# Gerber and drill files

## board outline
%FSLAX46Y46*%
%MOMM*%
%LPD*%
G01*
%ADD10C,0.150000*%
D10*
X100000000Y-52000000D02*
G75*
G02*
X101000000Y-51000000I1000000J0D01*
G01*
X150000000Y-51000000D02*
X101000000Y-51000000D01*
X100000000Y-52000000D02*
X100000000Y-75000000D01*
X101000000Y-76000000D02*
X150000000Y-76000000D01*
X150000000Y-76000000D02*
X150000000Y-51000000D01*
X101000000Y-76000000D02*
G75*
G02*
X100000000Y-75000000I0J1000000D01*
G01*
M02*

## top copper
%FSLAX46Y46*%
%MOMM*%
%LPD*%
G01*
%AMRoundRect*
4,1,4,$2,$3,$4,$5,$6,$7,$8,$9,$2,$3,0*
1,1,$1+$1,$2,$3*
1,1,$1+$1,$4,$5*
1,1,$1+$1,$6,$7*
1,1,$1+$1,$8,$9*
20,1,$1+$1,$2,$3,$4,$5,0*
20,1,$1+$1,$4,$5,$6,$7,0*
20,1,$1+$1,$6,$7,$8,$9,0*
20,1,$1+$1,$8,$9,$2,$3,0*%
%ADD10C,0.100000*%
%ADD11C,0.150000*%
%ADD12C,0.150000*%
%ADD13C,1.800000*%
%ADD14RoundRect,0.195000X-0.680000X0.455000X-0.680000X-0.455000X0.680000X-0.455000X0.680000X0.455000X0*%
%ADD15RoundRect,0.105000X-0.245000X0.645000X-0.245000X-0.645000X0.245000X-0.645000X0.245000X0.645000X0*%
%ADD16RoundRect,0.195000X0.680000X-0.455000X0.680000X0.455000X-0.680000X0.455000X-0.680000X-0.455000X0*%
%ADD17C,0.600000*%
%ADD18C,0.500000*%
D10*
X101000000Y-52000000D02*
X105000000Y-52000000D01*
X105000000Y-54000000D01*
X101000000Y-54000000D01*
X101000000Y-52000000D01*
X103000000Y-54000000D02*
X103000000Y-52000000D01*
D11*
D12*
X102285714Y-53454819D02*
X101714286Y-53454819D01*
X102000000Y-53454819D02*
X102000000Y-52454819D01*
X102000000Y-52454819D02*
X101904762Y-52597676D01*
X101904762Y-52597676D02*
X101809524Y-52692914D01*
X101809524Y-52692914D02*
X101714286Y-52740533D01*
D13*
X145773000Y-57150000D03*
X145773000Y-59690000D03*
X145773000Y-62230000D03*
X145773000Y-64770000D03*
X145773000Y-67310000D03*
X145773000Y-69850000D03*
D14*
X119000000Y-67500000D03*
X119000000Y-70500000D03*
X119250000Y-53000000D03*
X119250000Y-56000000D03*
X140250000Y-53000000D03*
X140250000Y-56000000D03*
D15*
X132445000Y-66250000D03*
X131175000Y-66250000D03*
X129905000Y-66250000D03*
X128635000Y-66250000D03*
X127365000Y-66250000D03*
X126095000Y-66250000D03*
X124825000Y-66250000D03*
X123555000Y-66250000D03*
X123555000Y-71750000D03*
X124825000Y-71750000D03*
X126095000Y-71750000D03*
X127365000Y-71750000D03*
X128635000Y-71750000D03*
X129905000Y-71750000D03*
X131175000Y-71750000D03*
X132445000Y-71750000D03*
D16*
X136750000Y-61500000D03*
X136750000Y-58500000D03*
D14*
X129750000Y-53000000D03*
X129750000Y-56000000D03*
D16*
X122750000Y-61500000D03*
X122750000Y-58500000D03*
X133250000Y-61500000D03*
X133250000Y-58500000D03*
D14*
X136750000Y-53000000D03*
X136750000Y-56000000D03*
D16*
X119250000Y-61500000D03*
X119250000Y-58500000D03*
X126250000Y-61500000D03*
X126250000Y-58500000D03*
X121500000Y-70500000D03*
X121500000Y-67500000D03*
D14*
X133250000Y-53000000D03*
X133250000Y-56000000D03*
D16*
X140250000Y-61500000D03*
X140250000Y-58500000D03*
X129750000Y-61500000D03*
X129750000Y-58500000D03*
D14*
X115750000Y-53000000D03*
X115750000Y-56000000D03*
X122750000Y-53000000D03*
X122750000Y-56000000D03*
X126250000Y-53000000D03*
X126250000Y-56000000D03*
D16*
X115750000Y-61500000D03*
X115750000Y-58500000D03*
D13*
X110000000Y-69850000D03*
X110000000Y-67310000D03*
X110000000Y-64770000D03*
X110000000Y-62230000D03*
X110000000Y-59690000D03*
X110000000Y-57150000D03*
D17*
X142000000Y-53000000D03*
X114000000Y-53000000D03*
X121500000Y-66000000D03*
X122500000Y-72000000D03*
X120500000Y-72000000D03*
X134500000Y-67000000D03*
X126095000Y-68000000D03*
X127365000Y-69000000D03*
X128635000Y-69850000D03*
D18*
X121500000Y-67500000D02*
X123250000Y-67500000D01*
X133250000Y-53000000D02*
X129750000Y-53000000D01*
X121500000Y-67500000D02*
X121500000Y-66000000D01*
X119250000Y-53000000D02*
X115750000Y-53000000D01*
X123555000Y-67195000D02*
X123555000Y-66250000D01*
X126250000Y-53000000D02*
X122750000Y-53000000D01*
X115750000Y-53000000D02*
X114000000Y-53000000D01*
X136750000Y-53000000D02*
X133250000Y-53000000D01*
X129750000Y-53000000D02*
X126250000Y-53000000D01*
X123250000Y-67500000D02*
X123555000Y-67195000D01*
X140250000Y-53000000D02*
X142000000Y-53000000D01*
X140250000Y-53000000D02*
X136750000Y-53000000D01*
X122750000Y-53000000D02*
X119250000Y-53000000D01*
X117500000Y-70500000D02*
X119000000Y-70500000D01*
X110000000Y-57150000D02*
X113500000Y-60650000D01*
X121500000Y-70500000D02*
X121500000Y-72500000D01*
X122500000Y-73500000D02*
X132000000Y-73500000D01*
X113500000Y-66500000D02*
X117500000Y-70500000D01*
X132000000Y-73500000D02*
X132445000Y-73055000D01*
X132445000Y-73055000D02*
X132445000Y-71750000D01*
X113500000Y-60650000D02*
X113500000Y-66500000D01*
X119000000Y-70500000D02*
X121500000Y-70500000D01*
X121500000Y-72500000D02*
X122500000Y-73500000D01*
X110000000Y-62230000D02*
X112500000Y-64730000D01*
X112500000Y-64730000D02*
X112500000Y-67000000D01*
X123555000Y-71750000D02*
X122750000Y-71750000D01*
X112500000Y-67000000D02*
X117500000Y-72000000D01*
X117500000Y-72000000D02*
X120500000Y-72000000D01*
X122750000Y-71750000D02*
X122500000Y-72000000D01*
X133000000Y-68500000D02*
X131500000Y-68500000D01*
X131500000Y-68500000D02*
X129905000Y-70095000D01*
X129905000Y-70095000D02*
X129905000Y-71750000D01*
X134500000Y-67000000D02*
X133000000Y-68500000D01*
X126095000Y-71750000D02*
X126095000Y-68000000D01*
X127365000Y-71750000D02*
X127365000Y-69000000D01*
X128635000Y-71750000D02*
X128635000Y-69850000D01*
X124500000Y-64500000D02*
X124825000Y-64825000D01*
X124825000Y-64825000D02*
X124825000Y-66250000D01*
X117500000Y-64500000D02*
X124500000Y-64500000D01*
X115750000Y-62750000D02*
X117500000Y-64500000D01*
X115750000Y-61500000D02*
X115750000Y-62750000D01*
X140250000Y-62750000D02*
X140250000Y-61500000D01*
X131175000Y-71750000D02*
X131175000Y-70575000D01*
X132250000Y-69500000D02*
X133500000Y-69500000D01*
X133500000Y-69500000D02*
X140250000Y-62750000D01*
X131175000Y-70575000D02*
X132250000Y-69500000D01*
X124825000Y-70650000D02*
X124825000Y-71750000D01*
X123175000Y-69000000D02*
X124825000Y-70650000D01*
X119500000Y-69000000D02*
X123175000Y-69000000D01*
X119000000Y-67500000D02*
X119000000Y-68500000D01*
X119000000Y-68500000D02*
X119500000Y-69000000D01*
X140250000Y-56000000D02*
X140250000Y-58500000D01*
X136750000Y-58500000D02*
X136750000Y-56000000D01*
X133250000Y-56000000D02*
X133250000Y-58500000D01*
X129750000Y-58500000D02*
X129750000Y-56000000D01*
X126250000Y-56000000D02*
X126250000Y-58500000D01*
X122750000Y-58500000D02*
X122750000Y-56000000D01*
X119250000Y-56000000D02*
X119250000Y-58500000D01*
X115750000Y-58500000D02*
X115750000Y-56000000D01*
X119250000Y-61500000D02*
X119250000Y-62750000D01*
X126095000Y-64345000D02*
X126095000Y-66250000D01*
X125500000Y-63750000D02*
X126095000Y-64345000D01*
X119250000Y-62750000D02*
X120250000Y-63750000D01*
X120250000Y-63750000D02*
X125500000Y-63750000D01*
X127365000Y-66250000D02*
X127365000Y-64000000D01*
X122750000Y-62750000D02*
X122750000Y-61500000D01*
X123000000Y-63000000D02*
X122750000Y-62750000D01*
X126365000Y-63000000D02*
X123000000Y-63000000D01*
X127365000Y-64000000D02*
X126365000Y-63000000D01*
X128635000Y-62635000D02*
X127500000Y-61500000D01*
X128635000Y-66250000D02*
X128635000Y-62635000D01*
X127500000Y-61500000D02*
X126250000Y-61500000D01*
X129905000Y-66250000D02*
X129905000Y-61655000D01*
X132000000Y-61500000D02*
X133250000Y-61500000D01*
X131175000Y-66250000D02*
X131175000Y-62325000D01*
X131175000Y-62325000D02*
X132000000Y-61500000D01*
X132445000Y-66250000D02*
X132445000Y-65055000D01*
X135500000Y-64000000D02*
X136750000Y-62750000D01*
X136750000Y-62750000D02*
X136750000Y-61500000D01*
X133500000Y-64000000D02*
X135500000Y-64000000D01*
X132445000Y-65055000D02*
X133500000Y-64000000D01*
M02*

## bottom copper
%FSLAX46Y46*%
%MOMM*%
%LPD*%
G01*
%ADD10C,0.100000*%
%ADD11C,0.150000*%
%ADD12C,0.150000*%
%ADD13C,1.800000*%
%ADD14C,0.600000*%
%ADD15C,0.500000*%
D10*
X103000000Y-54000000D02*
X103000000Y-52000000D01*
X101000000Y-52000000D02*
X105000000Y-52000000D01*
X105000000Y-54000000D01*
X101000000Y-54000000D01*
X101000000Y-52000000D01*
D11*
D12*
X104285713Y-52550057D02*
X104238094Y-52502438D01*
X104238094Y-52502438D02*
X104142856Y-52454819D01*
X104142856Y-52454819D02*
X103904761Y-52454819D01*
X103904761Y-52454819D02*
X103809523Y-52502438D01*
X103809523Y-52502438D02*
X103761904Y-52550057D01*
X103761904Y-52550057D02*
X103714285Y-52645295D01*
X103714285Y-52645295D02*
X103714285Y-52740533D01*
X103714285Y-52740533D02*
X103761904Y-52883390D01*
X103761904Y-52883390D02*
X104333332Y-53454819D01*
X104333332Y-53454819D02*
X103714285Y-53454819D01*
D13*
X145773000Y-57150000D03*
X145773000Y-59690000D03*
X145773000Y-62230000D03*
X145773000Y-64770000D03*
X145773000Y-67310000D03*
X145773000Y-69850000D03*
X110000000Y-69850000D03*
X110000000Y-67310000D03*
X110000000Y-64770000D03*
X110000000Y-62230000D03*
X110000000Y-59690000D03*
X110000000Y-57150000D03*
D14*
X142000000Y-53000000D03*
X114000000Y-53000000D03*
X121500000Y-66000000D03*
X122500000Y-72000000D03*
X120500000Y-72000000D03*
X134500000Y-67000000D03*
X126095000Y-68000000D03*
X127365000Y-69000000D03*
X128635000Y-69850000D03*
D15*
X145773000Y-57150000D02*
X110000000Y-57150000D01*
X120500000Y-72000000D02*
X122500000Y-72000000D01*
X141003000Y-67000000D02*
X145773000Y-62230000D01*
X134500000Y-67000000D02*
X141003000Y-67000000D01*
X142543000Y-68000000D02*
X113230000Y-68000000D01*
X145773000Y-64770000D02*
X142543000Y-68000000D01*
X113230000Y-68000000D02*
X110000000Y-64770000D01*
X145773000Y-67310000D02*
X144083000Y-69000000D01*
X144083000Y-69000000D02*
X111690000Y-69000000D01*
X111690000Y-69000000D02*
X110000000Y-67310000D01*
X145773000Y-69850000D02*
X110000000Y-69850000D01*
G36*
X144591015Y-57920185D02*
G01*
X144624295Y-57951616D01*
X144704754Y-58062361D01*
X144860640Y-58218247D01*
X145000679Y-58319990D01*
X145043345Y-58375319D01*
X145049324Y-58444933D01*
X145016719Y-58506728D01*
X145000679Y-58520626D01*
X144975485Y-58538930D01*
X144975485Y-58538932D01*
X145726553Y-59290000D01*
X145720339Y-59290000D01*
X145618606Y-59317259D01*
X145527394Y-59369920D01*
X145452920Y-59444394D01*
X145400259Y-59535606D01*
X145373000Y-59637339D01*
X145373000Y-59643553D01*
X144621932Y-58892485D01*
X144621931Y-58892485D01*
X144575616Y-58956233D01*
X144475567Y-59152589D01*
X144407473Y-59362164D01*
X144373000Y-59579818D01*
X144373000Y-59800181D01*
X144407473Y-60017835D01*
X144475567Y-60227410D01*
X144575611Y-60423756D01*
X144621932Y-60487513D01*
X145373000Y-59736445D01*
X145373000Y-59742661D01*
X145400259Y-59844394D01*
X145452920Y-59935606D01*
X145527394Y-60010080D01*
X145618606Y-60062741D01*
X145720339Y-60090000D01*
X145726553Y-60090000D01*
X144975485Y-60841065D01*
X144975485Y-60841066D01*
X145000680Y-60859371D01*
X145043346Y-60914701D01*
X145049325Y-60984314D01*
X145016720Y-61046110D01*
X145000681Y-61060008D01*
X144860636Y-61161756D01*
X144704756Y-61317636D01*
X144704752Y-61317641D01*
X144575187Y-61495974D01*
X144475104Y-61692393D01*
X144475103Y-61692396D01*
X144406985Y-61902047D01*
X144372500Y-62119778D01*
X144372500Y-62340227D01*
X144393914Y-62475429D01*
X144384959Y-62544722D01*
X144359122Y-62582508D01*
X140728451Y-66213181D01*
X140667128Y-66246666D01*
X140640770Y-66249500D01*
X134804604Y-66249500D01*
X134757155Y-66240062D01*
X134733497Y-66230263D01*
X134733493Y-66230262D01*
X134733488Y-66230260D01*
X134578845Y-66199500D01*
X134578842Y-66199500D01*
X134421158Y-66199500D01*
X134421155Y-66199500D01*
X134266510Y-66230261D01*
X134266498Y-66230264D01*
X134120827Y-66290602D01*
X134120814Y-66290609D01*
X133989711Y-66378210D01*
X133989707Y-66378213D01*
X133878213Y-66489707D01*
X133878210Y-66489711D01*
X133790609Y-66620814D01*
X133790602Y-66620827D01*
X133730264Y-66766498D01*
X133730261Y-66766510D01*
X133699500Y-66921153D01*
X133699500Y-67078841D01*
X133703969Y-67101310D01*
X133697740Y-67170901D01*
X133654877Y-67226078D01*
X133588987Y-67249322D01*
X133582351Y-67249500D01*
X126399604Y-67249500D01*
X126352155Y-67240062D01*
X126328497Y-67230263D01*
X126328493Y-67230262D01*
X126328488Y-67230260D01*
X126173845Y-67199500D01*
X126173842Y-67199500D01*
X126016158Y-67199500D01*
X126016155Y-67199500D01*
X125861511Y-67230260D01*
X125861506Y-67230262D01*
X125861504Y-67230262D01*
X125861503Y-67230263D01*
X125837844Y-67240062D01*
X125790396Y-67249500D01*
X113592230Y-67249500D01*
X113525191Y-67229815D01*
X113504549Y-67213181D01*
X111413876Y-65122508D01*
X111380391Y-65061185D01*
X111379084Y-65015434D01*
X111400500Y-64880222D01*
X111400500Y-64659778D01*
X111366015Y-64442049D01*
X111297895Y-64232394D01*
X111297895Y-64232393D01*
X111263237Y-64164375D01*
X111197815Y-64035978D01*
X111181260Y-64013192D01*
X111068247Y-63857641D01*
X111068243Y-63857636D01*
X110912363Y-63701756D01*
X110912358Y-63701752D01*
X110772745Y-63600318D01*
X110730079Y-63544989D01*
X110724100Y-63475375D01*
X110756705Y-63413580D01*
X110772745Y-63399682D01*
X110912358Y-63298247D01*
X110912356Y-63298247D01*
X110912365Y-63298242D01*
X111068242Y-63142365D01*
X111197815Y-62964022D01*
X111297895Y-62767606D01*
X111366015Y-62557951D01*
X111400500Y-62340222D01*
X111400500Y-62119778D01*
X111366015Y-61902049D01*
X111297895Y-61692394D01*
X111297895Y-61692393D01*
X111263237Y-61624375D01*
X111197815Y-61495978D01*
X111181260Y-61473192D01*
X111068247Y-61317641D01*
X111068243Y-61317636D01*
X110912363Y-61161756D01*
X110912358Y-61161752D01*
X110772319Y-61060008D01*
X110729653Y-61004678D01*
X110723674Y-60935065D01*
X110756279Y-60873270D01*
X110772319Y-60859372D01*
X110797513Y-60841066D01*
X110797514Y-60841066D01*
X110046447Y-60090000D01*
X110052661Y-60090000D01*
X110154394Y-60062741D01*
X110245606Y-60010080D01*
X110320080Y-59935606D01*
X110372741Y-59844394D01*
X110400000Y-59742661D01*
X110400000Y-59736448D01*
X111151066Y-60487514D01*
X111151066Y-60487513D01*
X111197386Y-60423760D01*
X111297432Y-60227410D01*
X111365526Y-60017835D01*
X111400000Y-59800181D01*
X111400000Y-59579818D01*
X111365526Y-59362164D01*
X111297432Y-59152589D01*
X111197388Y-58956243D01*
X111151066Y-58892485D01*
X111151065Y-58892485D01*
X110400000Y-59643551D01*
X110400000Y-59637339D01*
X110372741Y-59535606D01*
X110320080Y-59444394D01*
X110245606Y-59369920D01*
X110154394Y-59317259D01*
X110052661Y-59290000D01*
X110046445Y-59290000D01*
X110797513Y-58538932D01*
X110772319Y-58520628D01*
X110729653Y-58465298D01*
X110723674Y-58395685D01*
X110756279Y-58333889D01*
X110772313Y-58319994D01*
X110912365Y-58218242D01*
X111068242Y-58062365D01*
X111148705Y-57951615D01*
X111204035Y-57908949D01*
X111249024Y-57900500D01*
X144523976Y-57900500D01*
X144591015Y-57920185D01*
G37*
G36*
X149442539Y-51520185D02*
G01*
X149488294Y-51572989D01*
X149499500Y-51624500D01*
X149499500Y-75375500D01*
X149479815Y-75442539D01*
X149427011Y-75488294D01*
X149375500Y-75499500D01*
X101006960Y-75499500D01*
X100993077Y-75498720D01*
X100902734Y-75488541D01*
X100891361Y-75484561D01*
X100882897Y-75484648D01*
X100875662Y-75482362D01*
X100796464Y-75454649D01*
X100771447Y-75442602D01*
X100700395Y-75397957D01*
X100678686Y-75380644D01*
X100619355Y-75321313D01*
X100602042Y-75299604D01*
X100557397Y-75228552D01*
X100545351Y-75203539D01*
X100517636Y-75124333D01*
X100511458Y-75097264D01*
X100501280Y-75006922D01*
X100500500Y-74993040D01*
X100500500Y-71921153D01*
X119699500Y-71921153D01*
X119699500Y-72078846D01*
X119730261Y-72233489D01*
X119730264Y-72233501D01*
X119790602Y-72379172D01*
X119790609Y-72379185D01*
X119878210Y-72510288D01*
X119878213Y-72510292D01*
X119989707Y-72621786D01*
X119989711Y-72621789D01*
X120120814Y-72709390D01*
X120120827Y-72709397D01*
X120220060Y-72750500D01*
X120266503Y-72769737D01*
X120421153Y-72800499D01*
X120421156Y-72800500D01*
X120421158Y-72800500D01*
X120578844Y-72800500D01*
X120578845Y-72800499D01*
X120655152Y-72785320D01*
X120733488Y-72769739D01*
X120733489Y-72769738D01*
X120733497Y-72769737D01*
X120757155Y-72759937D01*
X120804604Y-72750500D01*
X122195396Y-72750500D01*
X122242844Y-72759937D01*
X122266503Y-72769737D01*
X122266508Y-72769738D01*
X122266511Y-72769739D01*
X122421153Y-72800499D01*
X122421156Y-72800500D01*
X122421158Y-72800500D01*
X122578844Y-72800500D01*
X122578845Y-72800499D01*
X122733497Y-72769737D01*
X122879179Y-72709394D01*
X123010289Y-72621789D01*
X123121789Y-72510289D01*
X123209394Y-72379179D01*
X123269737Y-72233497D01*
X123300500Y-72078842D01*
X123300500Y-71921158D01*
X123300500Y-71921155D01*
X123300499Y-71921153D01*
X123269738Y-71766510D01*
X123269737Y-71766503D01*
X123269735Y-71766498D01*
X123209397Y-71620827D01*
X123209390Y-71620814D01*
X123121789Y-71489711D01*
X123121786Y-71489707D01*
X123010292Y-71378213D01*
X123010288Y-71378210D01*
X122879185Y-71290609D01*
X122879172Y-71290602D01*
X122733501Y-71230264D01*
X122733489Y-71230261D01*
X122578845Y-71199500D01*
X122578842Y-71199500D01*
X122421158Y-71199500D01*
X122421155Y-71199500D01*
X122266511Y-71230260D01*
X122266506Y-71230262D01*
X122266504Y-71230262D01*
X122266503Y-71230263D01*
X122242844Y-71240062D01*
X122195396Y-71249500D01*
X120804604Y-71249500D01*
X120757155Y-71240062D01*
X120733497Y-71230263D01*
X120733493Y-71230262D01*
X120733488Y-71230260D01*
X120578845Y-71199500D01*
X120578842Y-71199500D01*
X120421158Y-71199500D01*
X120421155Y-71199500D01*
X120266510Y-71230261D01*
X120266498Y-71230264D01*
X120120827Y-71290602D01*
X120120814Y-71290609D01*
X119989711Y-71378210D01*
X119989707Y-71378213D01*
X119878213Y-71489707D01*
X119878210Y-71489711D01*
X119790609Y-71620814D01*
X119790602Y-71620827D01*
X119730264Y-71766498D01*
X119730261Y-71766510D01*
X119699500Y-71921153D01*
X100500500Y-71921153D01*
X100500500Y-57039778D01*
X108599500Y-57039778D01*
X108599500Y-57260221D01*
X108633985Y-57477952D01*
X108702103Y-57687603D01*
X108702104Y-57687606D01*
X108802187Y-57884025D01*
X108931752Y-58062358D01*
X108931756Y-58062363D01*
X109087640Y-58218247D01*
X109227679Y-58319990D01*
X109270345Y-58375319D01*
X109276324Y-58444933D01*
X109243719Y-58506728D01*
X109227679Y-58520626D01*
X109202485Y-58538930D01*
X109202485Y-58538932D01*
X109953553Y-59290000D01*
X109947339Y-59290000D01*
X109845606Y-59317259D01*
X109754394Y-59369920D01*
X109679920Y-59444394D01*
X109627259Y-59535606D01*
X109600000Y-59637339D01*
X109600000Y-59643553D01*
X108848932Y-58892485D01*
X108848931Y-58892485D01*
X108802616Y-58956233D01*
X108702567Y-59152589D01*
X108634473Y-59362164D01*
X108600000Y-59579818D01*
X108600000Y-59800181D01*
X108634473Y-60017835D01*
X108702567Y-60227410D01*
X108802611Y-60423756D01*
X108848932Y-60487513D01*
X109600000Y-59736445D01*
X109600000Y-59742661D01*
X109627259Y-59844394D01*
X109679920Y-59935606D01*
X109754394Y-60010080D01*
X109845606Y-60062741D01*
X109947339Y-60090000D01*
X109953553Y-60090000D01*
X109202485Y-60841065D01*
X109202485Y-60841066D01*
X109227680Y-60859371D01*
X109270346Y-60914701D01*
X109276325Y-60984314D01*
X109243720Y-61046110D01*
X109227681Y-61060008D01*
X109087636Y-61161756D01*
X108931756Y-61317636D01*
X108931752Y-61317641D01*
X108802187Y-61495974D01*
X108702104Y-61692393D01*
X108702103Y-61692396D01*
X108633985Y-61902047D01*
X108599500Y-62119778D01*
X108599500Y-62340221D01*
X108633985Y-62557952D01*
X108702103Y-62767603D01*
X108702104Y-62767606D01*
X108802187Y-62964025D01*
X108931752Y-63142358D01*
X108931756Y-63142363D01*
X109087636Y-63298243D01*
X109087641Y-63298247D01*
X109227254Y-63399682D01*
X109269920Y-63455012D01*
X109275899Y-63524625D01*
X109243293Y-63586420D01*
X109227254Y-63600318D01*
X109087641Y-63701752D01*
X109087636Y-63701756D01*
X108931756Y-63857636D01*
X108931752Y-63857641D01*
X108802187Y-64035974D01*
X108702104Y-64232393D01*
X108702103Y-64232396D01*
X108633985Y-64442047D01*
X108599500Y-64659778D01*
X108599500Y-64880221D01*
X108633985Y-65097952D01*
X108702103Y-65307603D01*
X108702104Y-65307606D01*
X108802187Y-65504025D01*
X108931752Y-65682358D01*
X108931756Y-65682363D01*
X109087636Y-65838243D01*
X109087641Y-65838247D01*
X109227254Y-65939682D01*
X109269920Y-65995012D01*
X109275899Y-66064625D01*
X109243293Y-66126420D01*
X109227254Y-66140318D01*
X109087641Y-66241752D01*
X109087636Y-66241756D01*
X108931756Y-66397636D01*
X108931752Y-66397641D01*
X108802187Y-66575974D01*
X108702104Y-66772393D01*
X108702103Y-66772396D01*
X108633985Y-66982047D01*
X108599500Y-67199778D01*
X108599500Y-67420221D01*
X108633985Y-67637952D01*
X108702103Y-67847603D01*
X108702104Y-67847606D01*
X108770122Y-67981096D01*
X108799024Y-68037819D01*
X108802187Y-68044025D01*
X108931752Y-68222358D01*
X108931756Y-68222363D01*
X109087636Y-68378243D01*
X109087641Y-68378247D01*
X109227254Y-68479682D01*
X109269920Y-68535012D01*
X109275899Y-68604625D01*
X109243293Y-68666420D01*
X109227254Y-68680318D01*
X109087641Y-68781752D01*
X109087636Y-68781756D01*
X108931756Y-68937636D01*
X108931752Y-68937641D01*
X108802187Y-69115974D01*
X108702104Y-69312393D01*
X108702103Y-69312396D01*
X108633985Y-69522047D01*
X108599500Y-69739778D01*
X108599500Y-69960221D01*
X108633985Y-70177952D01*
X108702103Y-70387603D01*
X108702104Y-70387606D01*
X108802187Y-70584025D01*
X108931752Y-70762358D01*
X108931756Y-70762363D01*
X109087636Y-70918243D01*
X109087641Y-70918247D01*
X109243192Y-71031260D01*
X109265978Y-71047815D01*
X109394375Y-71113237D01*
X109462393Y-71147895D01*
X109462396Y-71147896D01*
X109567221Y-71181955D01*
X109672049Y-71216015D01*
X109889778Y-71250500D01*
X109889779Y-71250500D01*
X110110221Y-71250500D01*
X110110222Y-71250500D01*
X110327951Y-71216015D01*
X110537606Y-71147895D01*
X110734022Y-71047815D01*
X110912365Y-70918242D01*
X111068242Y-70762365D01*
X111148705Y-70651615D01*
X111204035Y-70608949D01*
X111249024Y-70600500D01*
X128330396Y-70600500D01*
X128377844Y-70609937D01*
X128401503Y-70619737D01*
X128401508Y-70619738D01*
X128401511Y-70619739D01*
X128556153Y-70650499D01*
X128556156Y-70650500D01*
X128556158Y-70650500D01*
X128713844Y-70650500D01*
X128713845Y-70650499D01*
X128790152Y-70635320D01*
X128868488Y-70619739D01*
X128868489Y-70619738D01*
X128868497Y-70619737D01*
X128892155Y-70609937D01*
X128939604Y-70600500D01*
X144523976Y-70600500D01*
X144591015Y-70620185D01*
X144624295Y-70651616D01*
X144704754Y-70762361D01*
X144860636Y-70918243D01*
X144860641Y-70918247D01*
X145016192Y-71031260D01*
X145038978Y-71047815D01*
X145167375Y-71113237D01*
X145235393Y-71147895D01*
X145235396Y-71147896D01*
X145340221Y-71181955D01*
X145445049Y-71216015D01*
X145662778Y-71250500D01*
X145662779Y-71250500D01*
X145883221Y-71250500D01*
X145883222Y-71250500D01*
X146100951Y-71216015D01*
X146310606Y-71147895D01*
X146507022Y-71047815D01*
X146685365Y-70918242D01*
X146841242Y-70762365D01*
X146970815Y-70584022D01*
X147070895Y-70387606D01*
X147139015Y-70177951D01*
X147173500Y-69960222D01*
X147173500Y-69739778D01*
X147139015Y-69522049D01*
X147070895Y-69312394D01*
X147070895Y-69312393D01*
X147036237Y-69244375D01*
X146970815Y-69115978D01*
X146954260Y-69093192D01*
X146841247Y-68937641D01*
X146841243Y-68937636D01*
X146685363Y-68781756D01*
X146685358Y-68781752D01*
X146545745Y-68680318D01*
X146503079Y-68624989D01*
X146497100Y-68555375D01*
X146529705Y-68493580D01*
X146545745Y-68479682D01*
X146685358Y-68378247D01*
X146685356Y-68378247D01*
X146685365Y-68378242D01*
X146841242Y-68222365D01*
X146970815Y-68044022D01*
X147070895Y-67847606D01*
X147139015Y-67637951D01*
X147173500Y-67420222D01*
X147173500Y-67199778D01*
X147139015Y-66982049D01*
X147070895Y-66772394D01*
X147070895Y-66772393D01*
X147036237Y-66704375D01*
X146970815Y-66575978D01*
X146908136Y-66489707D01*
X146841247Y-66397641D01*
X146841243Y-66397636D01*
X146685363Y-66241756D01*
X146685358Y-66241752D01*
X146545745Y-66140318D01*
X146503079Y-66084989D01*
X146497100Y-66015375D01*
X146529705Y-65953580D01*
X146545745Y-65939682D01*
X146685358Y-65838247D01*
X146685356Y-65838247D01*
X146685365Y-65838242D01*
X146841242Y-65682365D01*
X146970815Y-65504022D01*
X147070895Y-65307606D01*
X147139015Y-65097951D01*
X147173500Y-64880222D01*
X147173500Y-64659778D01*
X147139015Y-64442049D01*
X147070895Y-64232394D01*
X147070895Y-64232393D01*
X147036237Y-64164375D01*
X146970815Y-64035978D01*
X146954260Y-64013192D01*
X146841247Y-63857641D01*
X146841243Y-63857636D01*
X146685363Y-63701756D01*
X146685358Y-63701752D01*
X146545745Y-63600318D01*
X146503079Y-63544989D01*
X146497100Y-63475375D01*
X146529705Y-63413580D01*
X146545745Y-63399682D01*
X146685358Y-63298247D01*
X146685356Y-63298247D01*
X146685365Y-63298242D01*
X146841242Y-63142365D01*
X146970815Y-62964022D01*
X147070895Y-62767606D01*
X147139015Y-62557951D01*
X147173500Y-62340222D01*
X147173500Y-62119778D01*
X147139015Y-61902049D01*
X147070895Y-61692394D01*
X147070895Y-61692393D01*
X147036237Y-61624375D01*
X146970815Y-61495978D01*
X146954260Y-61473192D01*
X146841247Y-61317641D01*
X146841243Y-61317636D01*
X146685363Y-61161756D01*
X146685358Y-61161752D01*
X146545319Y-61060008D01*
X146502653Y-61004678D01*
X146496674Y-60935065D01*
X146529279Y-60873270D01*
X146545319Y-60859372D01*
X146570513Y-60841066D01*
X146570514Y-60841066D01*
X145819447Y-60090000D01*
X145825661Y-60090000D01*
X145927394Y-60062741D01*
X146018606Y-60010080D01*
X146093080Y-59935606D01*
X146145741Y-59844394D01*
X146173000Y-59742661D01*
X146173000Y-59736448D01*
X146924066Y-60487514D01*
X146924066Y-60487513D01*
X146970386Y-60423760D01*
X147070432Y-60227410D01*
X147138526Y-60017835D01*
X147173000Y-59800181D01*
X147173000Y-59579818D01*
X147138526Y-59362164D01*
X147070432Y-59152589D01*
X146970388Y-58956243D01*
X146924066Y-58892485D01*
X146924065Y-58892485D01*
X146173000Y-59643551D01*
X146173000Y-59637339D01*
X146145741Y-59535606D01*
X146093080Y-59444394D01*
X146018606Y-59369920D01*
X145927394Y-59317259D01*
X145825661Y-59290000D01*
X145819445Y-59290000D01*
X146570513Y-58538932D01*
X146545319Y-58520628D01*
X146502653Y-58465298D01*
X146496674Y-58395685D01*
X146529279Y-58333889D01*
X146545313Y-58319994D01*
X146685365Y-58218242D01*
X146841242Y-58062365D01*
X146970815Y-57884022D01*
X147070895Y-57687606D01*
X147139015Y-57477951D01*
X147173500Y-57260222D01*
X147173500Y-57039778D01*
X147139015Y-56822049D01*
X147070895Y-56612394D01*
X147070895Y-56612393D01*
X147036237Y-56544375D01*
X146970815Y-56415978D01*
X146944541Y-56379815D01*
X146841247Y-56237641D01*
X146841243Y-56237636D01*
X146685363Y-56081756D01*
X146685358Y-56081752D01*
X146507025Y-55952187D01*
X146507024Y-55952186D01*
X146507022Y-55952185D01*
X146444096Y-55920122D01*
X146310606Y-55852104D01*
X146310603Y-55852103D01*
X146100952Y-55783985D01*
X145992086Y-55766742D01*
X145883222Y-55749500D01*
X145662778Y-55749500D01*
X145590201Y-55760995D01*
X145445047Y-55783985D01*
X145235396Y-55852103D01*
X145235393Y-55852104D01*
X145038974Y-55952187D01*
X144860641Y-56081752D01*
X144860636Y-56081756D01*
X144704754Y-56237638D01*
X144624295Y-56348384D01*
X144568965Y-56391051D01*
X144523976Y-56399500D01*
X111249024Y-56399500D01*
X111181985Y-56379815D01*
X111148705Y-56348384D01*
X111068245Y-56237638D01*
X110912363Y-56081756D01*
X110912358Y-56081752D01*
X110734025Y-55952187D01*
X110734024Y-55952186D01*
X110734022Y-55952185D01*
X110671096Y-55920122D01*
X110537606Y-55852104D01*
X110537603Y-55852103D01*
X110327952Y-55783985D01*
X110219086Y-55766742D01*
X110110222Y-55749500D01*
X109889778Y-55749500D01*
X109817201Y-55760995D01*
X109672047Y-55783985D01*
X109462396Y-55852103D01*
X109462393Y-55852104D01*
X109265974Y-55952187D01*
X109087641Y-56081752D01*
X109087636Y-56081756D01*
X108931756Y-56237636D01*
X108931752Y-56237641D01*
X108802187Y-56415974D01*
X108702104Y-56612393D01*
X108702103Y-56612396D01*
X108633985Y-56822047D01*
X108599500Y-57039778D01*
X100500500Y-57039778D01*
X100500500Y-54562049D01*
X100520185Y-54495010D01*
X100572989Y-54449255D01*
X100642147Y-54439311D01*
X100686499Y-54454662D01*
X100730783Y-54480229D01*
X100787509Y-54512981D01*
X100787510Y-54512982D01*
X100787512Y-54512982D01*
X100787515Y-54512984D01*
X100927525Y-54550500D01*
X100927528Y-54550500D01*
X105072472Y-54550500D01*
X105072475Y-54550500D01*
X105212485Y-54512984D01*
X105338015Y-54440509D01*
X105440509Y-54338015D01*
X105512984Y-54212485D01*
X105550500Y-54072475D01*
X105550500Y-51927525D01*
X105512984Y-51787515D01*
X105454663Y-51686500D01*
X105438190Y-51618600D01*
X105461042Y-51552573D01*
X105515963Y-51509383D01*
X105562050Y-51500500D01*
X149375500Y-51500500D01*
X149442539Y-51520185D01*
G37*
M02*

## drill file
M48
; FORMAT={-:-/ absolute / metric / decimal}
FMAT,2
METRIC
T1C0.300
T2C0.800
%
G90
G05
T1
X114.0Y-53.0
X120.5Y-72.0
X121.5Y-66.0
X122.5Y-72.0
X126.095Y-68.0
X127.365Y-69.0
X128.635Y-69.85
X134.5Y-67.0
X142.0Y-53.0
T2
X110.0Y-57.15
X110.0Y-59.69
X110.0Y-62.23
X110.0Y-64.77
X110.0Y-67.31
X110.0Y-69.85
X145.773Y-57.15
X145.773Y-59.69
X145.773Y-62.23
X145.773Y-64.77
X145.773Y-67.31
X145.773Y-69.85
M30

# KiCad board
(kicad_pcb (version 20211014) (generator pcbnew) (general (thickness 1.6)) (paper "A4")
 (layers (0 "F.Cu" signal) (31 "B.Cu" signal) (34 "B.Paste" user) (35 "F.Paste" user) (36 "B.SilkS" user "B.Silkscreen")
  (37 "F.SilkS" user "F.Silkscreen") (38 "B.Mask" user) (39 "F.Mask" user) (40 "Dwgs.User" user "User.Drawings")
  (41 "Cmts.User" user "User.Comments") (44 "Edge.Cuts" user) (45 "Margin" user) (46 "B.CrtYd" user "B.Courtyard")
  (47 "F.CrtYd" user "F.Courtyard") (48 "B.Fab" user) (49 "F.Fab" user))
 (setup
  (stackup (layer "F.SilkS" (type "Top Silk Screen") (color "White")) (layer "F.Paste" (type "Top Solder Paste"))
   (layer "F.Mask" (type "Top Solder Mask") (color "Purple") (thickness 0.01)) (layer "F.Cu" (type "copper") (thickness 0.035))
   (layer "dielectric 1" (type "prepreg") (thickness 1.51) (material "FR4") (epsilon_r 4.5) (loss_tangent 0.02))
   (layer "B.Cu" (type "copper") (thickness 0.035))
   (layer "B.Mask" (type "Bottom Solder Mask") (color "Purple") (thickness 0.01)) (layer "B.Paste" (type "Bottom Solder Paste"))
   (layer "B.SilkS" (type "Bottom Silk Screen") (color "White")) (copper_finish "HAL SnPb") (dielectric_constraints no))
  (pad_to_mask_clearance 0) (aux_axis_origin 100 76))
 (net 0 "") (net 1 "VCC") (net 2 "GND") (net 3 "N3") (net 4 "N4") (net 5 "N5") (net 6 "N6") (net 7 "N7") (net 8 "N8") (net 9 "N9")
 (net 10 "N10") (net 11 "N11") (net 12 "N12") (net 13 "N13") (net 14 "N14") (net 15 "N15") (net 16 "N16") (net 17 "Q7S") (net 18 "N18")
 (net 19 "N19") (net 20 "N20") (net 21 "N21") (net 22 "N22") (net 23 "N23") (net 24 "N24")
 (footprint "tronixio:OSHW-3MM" (layer "F.Cu") (at 148 73.5)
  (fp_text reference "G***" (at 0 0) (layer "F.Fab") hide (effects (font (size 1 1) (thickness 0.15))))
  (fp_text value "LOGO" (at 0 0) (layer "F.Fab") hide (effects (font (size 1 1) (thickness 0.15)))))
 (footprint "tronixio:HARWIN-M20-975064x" (layer "F.Cu") (at 145.773 57.15 -90)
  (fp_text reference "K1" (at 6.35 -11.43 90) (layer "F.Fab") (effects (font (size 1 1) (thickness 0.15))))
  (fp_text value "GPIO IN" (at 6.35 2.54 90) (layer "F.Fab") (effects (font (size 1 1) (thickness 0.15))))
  (pad "1" thru_hole circle locked (at 0 0 270) (size 1.8 1.8) (drill 0.8) (layers *.Cu *.Mask) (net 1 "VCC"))
  (pad "2" thru_hole circle (at 2.54 0 270) (size 1.8 1.8) (drill 0.8) (layers *.Cu *.Mask) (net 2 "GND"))
  (pad "3" thru_hole circle (at 5.08 0 270) (size 1.8 1.8) (drill 0.8) (layers *.Cu *.Mask) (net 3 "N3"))
  (pad "4" thru_hole circle (at 7.62 0 270) (size 1.8 1.8) (drill 0.8) (layers *.Cu *.Mask) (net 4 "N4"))
  (pad "5" thru_hole circle (at 10.16 0 270) (size 1.8 1.8) (drill 0.8) (layers *.Cu *.Mask) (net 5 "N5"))
  (pad "6" thru_hole circle (at 12.7 0 270) (size 1.8 1.8) (drill 0.8) (layers *.Cu *.Mask) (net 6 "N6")))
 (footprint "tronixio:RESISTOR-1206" (layer "F.Cu") (at 119 69 -90) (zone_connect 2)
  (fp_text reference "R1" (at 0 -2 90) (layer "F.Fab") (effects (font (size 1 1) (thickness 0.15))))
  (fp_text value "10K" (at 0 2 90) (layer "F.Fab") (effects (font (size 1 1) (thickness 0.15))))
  (pad "1" smd roundrect (at -1.5 0 270) (size 1.3 1.75) (layers "F.Cu" "F.Paste" "F.Mask") (roundrect_rratio 0.15) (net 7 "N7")
   (zone_connect 2))
  (pad "2" smd roundrect (at 1.5 0 270) (size 1.3 1.75) (layers "F.Cu" "F.Paste" "F.Mask") (roundrect_rratio 0.15) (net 1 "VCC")
   (zone_connect 2)))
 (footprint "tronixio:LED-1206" (layer "F.Cu") (at 119.25 54.5 -90) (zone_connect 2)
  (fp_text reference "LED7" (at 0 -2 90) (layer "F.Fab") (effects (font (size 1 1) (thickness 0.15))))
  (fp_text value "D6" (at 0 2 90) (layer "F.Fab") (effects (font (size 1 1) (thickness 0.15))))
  (pad "1" smd roundrect (at -1.5 0 270) (size 1.3 1.75) (layers "F.Cu" "F.Paste" "F.Mask") (roundrect_rratio 0.15) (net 2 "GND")
   (zone_connect 2))
  (pad "2" smd roundrect (at 1.5 0 270) (size 1.3 1.75) (layers "F.Cu" "F.Paste" "F.Mask") (roundrect_rratio 0.15) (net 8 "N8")
   (zone_connect 2)))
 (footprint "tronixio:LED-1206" (layer "F.Cu") (at 140.25 54.5 -90) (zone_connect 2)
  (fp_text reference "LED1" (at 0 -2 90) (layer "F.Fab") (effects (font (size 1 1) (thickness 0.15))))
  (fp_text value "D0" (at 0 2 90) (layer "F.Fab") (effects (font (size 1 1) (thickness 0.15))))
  (pad "1" smd roundrect (at -1.5 0 270) (size 1.3 1.75) (layers "F.Cu" "F.Paste" "F.Mask") (roundrect_rratio 0.15) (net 2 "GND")
   (zone_connect 2))
  (pad "2" smd roundrect (at 1.5 0 270) (size 1.3 1.75) (layers "F.Cu" "F.Paste" "F.Mask") (roundrect_rratio 0.15) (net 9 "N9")
   (zone_connect 2)))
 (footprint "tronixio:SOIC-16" (layer "F.Cu") (at 128 69 -90)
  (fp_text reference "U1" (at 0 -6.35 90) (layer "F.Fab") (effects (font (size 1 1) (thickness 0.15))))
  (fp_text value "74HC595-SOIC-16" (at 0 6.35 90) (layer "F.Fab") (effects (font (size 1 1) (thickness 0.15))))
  (pad "1" smd roundrect (at -2.75 -4.445 270) (size 1.5 0.7) (layers "F.Cu" "F.Paste" "F.Mask") (roundrect_rratio 0.15) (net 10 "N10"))
  (pad "2" smd roundrect (at -2.75 -3.175 270) (size 1.5 0.7) (layers "F.Cu" "F.Paste" "F.Mask") (roundrect_rratio 0.15) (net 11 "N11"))
  (pad "3" smd roundrect (at -2.75 -1.905 270) (size 1.5 0.7) (layers "F.Cu" "F.Paste" "F.Mask") (roundrect_rratio 0.15) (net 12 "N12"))
  (pad "4" smd roundrect (at -2.75 -0.635 270) (size 1.5 0.7) (layers "F.Cu" "F.Paste" "F.Mask") (roundrect_rratio 0.15) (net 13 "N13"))
  (pad "5" smd roundrect (at -2.75 0.635 270) (size 1.5 0.7) (layers "F.Cu" "F.Paste" "F.Mask") (roundrect_rratio 0.15) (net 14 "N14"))
  (pad "6" smd roundrect (at -2.75 1.905 270) (size 1.5 0.7) (layers "F.Cu" "F.Paste" "F.Mask") (roundrect_rratio 0.15) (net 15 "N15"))
  (pad "7" smd roundrect (at -2.75 3.175 270) (size 1.5 0.7) (layers "F.Cu" "F.Paste" "F.Mask") (roundrect_rratio 0.15) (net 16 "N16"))
  (pad "8" smd roundrect (at -2.75 4.445 270) (size 1.5 0.7) (layers "F.Cu" "F.Paste" "F.Mask") (roundrect_rratio 0.15) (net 2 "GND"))
  (pad "9" smd roundrect (at 2.75 4.445 270) (size 1.5 0.7) (layers "F.Cu" "F.Paste" "F.Mask") (roundrect_rratio 0.15) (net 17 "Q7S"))
  (pad "10" smd roundrect (at 2.75 3.175 270) (size 1.5 0.7) (layers "F.Cu" "F.Paste" "F.Mask") (roundrect_rratio 0.15) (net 7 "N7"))
  (pad "11" smd roundrect (at 2.75 1.905 270) (size 1.5 0.7) (layers "F.Cu" "F.Paste" "F.Mask") (roundrect_rratio 0.15) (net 4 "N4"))
  (pad "12" smd roundrect (at 2.75 0.635 270) (size 1.5 0.7) (layers "F.Cu" "F.Paste" "F.Mask") (roundrect_rratio 0.15) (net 5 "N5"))
  (pad "13" smd roundrect (at 2.75 -0.635 270) (size 1.5 0.7) (layers "F.Cu" "F.Paste" "F.Mask") (roundrect_rratio 0.15) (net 6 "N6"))
  (pad "14" smd roundrect (at 2.75 -1.905 270) (size 1.5 0.7) (layers "F.Cu" "F.Paste" "F.Mask") (roundrect_rratio 0.15) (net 3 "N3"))
  (pad "15" smd roundrect (at 2.75 -3.175 270) (size 1.5 0.7) (layers "F.Cu" "F.Paste" "F.Mask") (roundrect_rratio 0.15) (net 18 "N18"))
  (pad "16" smd roundrect (at 2.75 -4.445 270) (size 1.5 0.7) (layers "F.Cu" "F.Paste" "F.Mask") (roundrect_rratio 0.15) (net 1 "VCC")))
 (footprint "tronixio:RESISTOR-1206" (layer "F.Cu") (at 136.75 60 90) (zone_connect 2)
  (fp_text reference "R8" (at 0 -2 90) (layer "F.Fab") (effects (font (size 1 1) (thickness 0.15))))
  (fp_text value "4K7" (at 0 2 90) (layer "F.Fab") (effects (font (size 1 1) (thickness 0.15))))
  (pad "1" smd roundrect (at -1.5 0 90) (size 1.3 1.75) (layers "F.Cu" "F.Paste" "F.Mask") (roundrect_rratio 0.15) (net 10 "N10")
   (zone_connect 2))
  (pad "2" smd roundrect (at 1.5 0 90) (size 1.3 1.75) (layers "F.Cu" "F.Paste" "F.Mask") (roundrect_rratio 0.15) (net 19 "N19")
   (zone_connect 2)))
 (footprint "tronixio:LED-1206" (layer "F.Cu") (at 129.75 54.5 -90) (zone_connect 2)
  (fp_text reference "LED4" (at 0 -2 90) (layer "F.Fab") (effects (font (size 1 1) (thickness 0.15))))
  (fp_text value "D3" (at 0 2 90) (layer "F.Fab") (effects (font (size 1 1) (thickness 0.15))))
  (pad "1" smd roundrect (at -1.5 0 270) (size 1.3 1.75) (layers "F.Cu" "F.Paste" "F.Mask") (roundrect_rratio 0.15) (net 2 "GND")
   (zone_connect 2))
  (pad "2" smd roundrect (at 1.5 0 270) (size 1.3 1.75) (layers "F.Cu" "F.Paste" "F.Mask") (roundrect_rratio 0.15) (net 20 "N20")
   (zone_connect 2)))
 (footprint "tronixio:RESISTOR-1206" (layer "F.Cu") (at 122.75 60 90) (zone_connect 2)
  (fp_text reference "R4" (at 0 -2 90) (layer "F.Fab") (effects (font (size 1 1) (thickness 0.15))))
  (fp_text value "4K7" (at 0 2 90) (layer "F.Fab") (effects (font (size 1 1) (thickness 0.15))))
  (pad "1" smd roundrect (at -1.5 0 90) (size 1.3 1.75) (layers "F.Cu" "F.Paste" "F.Mask") (roundrect_rratio 0.15) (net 14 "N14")
   (zone_connect 2))
  (pad "2" smd roundrect (at 1.5 0 90) (size 1.3 1.75) (layers "F.Cu" "F.Paste" "F.Mask") (roundrect_rratio 0.15) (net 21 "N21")
   (zone_connect 2)))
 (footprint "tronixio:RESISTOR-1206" (layer "F.Cu") (at 133.25 60 90) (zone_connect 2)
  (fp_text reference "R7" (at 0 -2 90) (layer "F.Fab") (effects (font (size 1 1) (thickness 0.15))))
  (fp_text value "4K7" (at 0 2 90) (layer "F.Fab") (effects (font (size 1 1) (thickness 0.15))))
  (pad "1" smd roundrect (at -1.5 0 90) (size 1.3 1.75) (layers "F.Cu" "F.Paste" "F.Mask") (roundrect_rratio 0.15) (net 11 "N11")
   (zone_connect 2))
  (pad "2" smd roundrect (at 1.5 0 90) (size 1.3 1.75) (layers "F.Cu" "F.Paste" "F.Mask") (roundrect_rratio 0.15) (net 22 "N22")
   (zone_connect 2)))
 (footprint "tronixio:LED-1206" (layer "F.Cu") (at 136.75 54.5 -90) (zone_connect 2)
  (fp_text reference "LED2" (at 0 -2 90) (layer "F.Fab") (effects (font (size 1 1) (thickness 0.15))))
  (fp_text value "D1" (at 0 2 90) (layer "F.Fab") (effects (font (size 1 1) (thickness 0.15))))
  (pad "1" smd roundrect (at -1.5 0 270) (size 1.3 1.75) (layers "F.Cu" "F.Paste" "F.Mask") (roundrect_rratio 0.15) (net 2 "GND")
   (zone_connect 2))
  (pad "2" smd roundrect (at 1.5 0 270) (size 1.3 1.75) (layers "F.Cu" "F.Paste" "F.Mask") (roundrect_rratio 0.15) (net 19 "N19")
   (zone_connect 2)))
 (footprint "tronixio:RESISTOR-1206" (layer "F.Cu") (at 119.25 60 90) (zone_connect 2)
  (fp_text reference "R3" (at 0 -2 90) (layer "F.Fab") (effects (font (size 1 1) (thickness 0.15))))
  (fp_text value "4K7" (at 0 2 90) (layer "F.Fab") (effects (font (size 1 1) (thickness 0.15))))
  (pad "1" smd roundrect (at -1.5 0 90) (size 1.3 1.75) (layers "F.Cu" "F.Paste" "F.Mask") (roundrect_rratio 0.15) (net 15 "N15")
   (zone_connect 2))
  (pad "2" smd roundrect (at 1.5 0 90) (size 1.3 1.75) (layers "F.Cu" "F.Paste" "F.Mask") (roundrect_rratio 0.15) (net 8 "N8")
   (zone_connect 2)))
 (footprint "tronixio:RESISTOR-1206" (layer "F.Cu") (at 126.25 60 90) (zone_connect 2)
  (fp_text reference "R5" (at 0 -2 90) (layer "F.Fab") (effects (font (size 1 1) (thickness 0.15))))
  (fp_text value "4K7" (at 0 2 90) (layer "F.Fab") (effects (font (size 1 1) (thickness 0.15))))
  (pad "1" smd roundrect (at -1.5 0 90) (size 1.3 1.75) (layers "F.Cu" "F.Paste" "F.Mask") (roundrect_rratio 0.15) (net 13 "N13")
   (zone_connect 2))
  (pad "2" smd roundrect (at 1.5 0 90) (size 1.3 1.75) (layers "F.Cu" "F.Paste" "F.Mask") (roundrect_rratio 0.15) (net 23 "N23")
   (zone_connect 2)))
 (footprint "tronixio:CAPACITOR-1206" (layer "F.Cu") (at 121.5 69 90) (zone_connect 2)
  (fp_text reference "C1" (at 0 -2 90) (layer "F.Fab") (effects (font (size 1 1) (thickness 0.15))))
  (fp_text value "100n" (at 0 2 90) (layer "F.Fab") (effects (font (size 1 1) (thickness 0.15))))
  (pad "1" smd roundrect (at -1.5 0 90) (size 1.3 1.75) (layers "F.Cu" "F.Paste" "F.Mask") (roundrect_rratio 0.15) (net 1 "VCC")
   (zone_connect 2))
  (pad "2" smd roundrect (at 1.5 0 90) (size 1.3 1.75) (layers "F.Cu" "F.Paste" "F.Mask") (roundrect_rratio 0.15) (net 2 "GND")
   (zone_connect 2)))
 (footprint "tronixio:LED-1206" (layer "F.Cu") (at 133.25 54.5 -90) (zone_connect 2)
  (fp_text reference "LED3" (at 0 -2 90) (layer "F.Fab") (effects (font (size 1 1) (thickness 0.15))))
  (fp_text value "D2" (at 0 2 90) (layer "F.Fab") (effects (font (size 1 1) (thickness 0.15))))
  (pad "1" smd roundrect (at -1.5 0 270) (size 1.3 1.75) (layers "F.Cu" "F.Paste" "F.Mask") (roundrect_rratio 0.15) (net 2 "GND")
   (zone_connect 2))
  (pad "2" smd roundrect (at 1.5 0 270) (size 1.3 1.75) (layers "F.Cu" "F.Paste" "F.Mask") (roundrect_rratio 0.15) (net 22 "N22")
   (zone_connect 2)))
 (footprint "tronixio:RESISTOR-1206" (layer "F.Cu") (at 140.25 60 90) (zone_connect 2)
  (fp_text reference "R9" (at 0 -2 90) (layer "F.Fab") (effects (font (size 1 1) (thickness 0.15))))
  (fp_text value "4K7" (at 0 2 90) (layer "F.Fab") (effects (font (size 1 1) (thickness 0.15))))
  (pad "1" smd roundrect (at -1.5 0 90) (size 1.3 1.75) (layers "F.Cu" "F.Paste" "F.Mask") (roundrect_rratio 0.15) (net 18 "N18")
   (zone_connect 2))
  (pad "2" smd roundrect (at 1.5 0 90) (size 1.3 1.75) (layers "F.Cu" "F.Paste" "F.Mask") (roundrect_rratio 0.15) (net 9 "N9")
   (zone_connect 2)))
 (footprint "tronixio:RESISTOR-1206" (layer "F.Cu") (at 129.75 60 90) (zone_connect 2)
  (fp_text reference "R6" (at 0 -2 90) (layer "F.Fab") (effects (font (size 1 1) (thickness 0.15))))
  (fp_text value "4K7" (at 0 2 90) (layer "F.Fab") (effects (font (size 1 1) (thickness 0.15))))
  (pad "1" smd roundrect (at -1.5 0 90) (size 1.3 1.75) (layers "F.Cu" "F.Paste" "F.Mask") (roundrect_rratio 0.15) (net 12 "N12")
   (zone_connect 2))
  (pad "2" smd roundrect (at 1.5 0 90) (size 1.3 1.75) (layers "F.Cu" "F.Paste" "F.Mask") (roundrect_rratio 0.15) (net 20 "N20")
   (zone_connect 2)))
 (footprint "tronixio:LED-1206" (layer "F.Cu") (at 115.75 54.5 -90) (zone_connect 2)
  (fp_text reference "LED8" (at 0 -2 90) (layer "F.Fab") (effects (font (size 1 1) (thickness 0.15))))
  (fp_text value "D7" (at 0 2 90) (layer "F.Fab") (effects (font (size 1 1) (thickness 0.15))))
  (pad "1" smd roundrect (at -1.5 0 270) (size 1.3 1.75) (layers "F.Cu" "F.Paste" "F.Mask") (roundrect_rratio 0.15) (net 2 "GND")
   (zone_connect 2))
  (pad "2" smd roundrect (at 1.5 0 270) (size 1.3 1.75) (layers "F.Cu" "F.Paste" "F.Mask") (roundrect_rratio 0.15) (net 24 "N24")
   (zone_connect 2)))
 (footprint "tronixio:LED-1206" (layer "F.Cu") (at 122.75 54.5 -90) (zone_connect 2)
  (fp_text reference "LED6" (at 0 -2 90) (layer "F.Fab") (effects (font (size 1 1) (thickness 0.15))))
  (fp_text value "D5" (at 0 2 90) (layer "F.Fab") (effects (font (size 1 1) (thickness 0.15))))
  (pad "1" smd roundrect (at -1.5 0 270) (size 1.3 1.75) (layers "F.Cu" "F.Paste" "F.Mask") (roundrect_rratio 0.15) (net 2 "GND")
   (zone_connect 2))
  (pad "2" smd roundrect (at 1.5 0 270) (size 1.3 1.75) (layers "F.Cu" "F.Paste" "F.Mask") (roundrect_rratio 0.15) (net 21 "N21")
   (zone_connect 2)))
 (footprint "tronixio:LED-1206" (layer "F.Cu") (at 126.25 54.5 -90) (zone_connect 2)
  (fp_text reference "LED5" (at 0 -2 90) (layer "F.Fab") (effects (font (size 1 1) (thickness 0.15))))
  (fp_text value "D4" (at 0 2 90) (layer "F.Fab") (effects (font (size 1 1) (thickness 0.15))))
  (pad "1" smd roundrect (at -1.5 0 270) (size 1.3 1.75) (layers "F.Cu" "F.Paste" "F.Mask") (roundrect_rratio 0.15) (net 2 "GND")
   (zone_connect 2))
  (pad "2" smd roundrect (at 1.5 0 270) (size 1.3 1.75) (layers "F.Cu" "F.Paste" "F.Mask") (roundrect_rratio 0.15) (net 23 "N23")
   (zone_connect 2)))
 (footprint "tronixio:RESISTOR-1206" (layer "F.Cu") (at 115.75 60 90) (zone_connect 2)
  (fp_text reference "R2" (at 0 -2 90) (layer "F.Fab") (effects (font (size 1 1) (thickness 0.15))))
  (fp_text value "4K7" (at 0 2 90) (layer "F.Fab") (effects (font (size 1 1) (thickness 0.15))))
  (pad "1" smd roundrect (at -1.5 0 90) (size 1.3 1.75) (layers "F.Cu" "F.Paste" "F.Mask") (roundrect_rratio 0.15) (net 16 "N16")
   (zone_connect 2))
  (pad "2" smd roundrect (at 1.5 0 90) (size 1.3 1.75) (layers "F.Cu" "F.Paste" "F.Mask") (roundrect_rratio 0.15) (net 24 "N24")
   (zone_connect 2)))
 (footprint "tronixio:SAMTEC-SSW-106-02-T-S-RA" (layer "F.Cu") (at 110 69.85 90)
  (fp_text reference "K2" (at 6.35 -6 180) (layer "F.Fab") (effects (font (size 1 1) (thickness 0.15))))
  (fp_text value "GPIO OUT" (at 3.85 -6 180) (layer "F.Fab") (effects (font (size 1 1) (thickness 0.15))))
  (pad "1" thru_hole circle locked (at 0 0 90) (size 1.8 1.8) (drill 0.8) (layers *.Cu *.Mask) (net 6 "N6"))
  (pad "2" thru_hole circle locked (at 2.54 0 90) (size 1.8 1.8) (drill 0.8) (layers *.Cu *.Mask) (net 5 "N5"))
  (pad "3" thru_hole circle locked (at 5.08 0 90) (size 1.8 1.8) (drill 0.8) (layers *.Cu *.Mask) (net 4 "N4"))
  (pad "4" thru_hole circle locked (at 7.62 0 90) (size 1.8 1.8) (drill 0.8) (layers *.Cu *.Mask) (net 17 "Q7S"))
  (pad "5" thru_hole circle locked (at 10.16 0 90) (size 1.8 1.8) (drill 0.8) (layers *.Cu *.Mask) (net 2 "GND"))
  (pad "6" thru_hole circle locked (at 12.7 0 90) (size 1.8 1.8) (drill 0.8) (layers *.Cu *.Mask) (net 1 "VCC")))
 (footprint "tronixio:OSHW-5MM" (layer "B.Cu") (at 132 57.5 180)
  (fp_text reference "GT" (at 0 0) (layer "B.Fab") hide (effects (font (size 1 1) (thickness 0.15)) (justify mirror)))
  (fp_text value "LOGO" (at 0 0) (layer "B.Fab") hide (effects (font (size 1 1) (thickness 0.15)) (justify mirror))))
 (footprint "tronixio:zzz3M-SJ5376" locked (layer "B.Cu") (at 116.5 63.5 180)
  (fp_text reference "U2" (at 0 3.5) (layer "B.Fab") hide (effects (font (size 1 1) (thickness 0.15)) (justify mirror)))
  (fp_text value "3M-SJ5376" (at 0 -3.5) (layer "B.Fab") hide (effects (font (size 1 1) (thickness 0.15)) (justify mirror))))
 (gr_rect (start 101 54) (end 105 52) (layer "F.Cu") (width 0.1) (fill none))
 (gr_line (start 103 54) (end 103 52) (layer "F.Cu") (width 0.1))
 (gr_line (start 103 54) (end 103 52) (layer "B.Cu") (width 0.1))
 (gr_rect (start 101 54) (end 105 52) (layer "B.Cu") (width 0.1) (fill none))
 (gr_arc (start 100 52) (mid 100.292893 51.292893) (end 101 51) (layer "Edge.Cuts") (width 0.15))
 (gr_line (start 150 51) (end 101 51) (layer "Edge.Cuts") (width 0.15))
 (gr_line (start 100 52) (end 100 75) (layer "Edge.Cuts") (width 0.15))
 (gr_line (start 101 76) (end 150 76) (layer "Edge.Cuts") (width 0.15))
 (gr_line (start 150 76) (end 150 51) (layer "Edge.Cuts") (width 0.15))
 (gr_arc (start 101 76) (mid 100.292893 75.707107) (end 100 75) (layer "Edge.Cuts") (width 0.15))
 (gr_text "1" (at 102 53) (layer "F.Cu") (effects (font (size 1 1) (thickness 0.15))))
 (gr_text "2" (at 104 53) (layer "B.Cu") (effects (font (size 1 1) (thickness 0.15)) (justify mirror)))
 (segment (start 121.5 67.5) (end 123.25 67.5) (width 0.5) (layer "F.Cu") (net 2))
 (segment (start 133.25 53) (end 129.75 53) (width 0.5) (layer "F.Cu") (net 2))
 (segment (start 121.5 67.5) (end 121.5 66) (width 0.5) (layer "F.Cu") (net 2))
 (segment (start 119.25 53) (end 115.75 53) (width 0.5) (layer "F.Cu") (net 2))
 (segment (start 123.555 67.195) (end 123.555 66.25) (width 0.5) (layer "F.Cu") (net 2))
 (segment (start 126.25 53) (end 122.75 53) (width 0.5) (layer "F.Cu") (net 2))
 (segment (start 115.75 53) (end 114 53) (width 0.5) (layer "F.Cu") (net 2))
 (segment (start 136.75 53) (end 133.25 53) (width 0.5) (layer "F.Cu") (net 2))
 (segment (start 129.75 53) (end 126.25 53) (width 0.5) (layer "F.Cu") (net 2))
 (segment (start 123.25 67.5) (end 123.555 67.195) (width 0.5) (layer "F.Cu") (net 2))
 (segment (start 140.25 53) (end 142 53) (width 0.5) (layer "F.Cu") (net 2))
 (segment (start 140.25 53) (end 136.75 53) (width 0.5) (layer "F.Cu") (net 2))
 (segment (start 122.75 53) (end 119.25 53) (width 0.5) (layer "F.Cu") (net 2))
 (via (at 142 53) (size 0.6) (drill 0.3) (layers "F.Cu" "B.Cu") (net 2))
 (via (at 114 53) (size 0.6) (drill 0.3) (layers "F.Cu" "B.Cu") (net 2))
 (via (at 121.5 66) (size 0.6) (drill 0.3) (layers "F.Cu" "B.Cu") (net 2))
 (segment (start 117.5 70.5) (end 119 70.5) (width 0.5) (layer "F.Cu") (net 1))
 (segment (start 110 57.15) (end 113.5 60.65) (width 0.5) (layer "F.Cu") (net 1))
 (segment (start 121.5 70.5) (end 121.5 72.5) (width 0.5) (layer "F.Cu") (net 1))
 (segment (start 122.5 73.5) (end 132 73.5) (width 0.5) (layer "F.Cu") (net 1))
 (segment (start 113.5 66.5) (end 117.5 70.5) (width 0.5) (layer "F.Cu") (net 1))
 (segment (start 132 73.5) (end 132.445 73.055) (width 0.5) (layer "F.Cu") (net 1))
 (segment (start 132.445 73.055) (end 132.445 71.75) (width 0.5) (layer "F.Cu") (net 1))
 (segment (start 113.5 60.65) (end 113.5 66.5) (width 0.5) (layer "F.Cu") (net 1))
 (segment (start 119 70.5) (end 121.5 70.5) (width 0.5) (layer "F.Cu") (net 1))
 (segment (start 121.5 72.5) (end 122.5 73.5) (width 0.5) (layer "F.Cu") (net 1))
 (segment (start 145.773 57.15) (end 110 57.15) (width 0.5) (layer "B.Cu") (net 1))
 (segment (start 110 62.23) (end 112.5 64.73) (width 0.5) (layer "F.Cu") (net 17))
 (segment (start 112.5 64.73) (end 112.5 67) (width 0.5) (layer "F.Cu") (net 17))
 (segment (start 123.555 71.75) (end 122.75 71.75) (width 0.5) (layer "F.Cu") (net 17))
 (segment (start 112.5 67) (end 117.5 72) (width 0.5) (layer "F.Cu") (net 17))
 (segment (start 117.5 72) (end 120.5 72) (width 0.5) (layer "F.Cu") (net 17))
 (segment (start 122.75 71.75) (end 122.5 72) (width 0.5) (layer "F.Cu") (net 17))
 (via (at 122.5 72) (size 0.6) (drill 0.3) (layers "F.Cu" "B.Cu") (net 17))
 (via (at 120.5 72) (size 0.6) (drill 0.3) (layers "F.Cu" "B.Cu") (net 17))
 (segment (start 120.5 72) (end 122.5 72) (width 0.5) (layer "B.Cu") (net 17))
 (segment (start 133 68.5) (end 131.5 68.5) (width 0.5) (layer "F.Cu") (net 3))
 (segment (start 131.5 68.5) (end 129.905 70.095) (width 0.5) (layer "F.Cu") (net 3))
 (segment (start 129.905 70.095) (end 129.905 71.75) (width 0.5) (layer "F.Cu") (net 3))
 (segment (start 134.5 67) (end 133 68.5) (width 0.5) (layer "F.Cu") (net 3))
 (via (at 134.5 67) (size 0.6) (drill 0.3) (layers "F.Cu" "B.Cu") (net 3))
 (segment (start 141.003 67) (end 145.773 62.23) (width 0.5) (layer "B.Cu") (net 3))
 (segment (start 134.5 67) (end 141.003 67) (width 0.5) (layer "B.Cu") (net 3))
 (segment (start 126.095 71.75) (end 126.095 68) (width 0.5) (layer "F.Cu") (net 4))
 (via (at 126.095 68) (size 0.6) (drill 0.3) (layers "F.Cu" "B.Cu") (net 4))
 (segment (start 142.543 68) (end 113.23 68) (width 0.5) (layer "B.Cu") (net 4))
 (segment (start 145.773 64.77) (end 142.543 68) (width 0.5) (layer "B.Cu") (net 4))
 (segment (start 113.23 68) (end 110 64.77) (width 0.5) (layer "B.Cu") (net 4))
 (segment (start 127.365 71.75) (end 127.365 69) (width 0.5) (layer "F.Cu") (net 5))
 (via (at 127.365 69) (size 0.6) (drill 0.3) (layers "F.Cu" "B.Cu") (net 5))
 (segment (start 145.773 67.31) (end 144.083 69) (width 0.5) (layer "B.Cu") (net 5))
 (segment (start 144.083 69) (end 111.69 69) (width 0.5) (layer "B.Cu") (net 5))
 (segment (start 111.69 69) (end 110 67.31) (width 0.5) (layer "B.Cu") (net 5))
 (segment (start 128.635 71.75) (end 128.635 69.85) (width 0.5) (layer "F.Cu") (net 6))
 (via (at 128.635 69.85) (size 0.6) (drill 0.3) (layers "F.Cu" "B.Cu") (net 6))
 (segment (start 145.773 69.85) (end 110 69.85) (width 0.5) (layer "B.Cu") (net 6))
 (segment (start 124.5 64.5) (end 124.825 64.825) (width 0.5) (layer "F.Cu") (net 16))
 (segment (start 124.825 64.825) (end 124.825 66.25) (width 0.5) (layer "F.Cu") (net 16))
 (segment (start 117.5 64.5) (end 124.5 64.5) (width 0.5) (layer "F.Cu") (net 16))
 (segment (start 115.75 62.75) (end 117.5 64.5) (width 0.5) (layer "F.Cu") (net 16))
 (segment (start 115.75 61.5) (end 115.75 62.75) (width 0.5) (layer "F.Cu") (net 16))
 (segment (start 140.25 62.75) (end 140.25 61.5) (width 0.5) (layer "F.Cu") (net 18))
 (segment (start 131.175 71.75) (end 131.175 70.575) (width 0.5) (layer "F.Cu") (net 18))
 (segment (start 132.25 69.5) (end 133.5 69.5) (width 0.5) (layer "F.Cu") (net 18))
 (segment (start 133.5 69.5) (end 140.25 62.75) (width 0.5) (layer "F.Cu") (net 18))
 (segment (start 131.175 70.575) (end 132.25 69.5) (width 0.5) (layer "F.Cu") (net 18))
 (segment (start 124.825 70.65) (end 124.825 71.75) (width 0.5) (layer "F.Cu") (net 7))
 (segment (start 123.175 69) (end 124.825 70.65) (width 0.5) (layer "F.Cu") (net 7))
 (segment (start 119.5 69) (end 123.175 69) (width 0.5) (layer "F.Cu") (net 7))
 (segment (start 119 67.5) (end 119 68.5) (width 0.5) (layer "F.Cu") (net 7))
 (segment (start 119 68.5) (end 119.5 69) (width 0.5) (layer "F.Cu") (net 7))
 (segment (start 140.25 56) (end 140.25 58.5) (width 0.5) (layer "F.Cu") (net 9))
 (segment (start 136.75 58.5) (end 136.75 56) (width 0.5) (layer "F.Cu") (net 19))
 (segment (start 133.25 56) (end 133.25 58.5) (width 0.5) (layer "F.Cu") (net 22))
 (segment (start 129.75 58.5) (end 129.75 56) (width 0.5) (layer "F.Cu") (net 20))
 (segment (start 126.25 56) (end 126.25 58.5) (width 0.5) (layer "F.Cu") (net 23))
 (segment (start 122.75 58.5) (end 122.75 56) (width 0.5) (layer "F.Cu") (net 21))
 (segment (start 119.25 56) (end 119.25 58.5) (width 0.5) (layer "F.Cu") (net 8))
 (segment (start 115.75 58.5) (end 115.75 56) (width 0.5) (layer "F.Cu") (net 24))
 (segment (start 119.25 61.5) (end 119.25 62.75) (width 0.5) (layer "F.Cu") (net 15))
 (segment (start 126.095 64.345) (end 126.095 66.25) (width 0.5) (layer "F.Cu") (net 15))
 (segment (start 125.5 63.75) (end 126.095 64.345) (width 0.5) (layer "F.Cu") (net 15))
 (segment (start 119.25 62.75) (end 120.25 63.75) (width 0.5) (layer "F.Cu") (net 15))
 (segment (start 120.25 63.75) (end 125.5 63.75) (width 0.5) (layer "F.Cu") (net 15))
 (segment (start 127.365 66.25) (end 127.365 64) (width 0.5) (layer "F.Cu") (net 14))
 (segment (start 122.75 62.75) (end 122.75 61.5) (width 0.5) (layer "F.Cu") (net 14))
 (segment (start 123 63) (end 122.75 62.75) (width 0.5) (layer "F.Cu") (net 14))
 (segment (start 126.365 63) (end 123 63) (width 0.5) (layer "F.Cu") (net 14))
 (segment (start 127.365 64) (end 126.365 63) (width 0.5) (layer "F.Cu") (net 14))
 (segment (start 128.635 62.635) (end 127.5 61.5) (width 0.5) (layer "F.Cu") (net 13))
 (segment (start 128.635 66.25) (end 128.635 62.635) (width 0.5) (layer "F.Cu") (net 13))
 (segment (start 127.5 61.5) (end 126.25 61.5) (width 0.5) (layer "F.Cu") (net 13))
 (segment (start 129.905 66.25) (end 129.905 61.655) (width 0.5) (layer "F.Cu") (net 12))
 (segment (start 132 61.5) (end 133.25 61.5) (width 0.5) (layer "F.Cu") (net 11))
 (segment (start 131.175 66.25) (end 131.175 62.325) (width 0.5) (layer "F.Cu") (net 11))
 (segment (start 131.175 62.325) (end 132 61.5) (width 0.5) (layer "F.Cu") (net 11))
 (segment (start 132.445 66.25) (end 132.445 65.055) (width 0.5) (layer "F.Cu") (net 10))
 (segment (start 135.5 64) (end 136.75 62.75) (width 0.5) (layer "F.Cu") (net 10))
 (segment (start 136.75 62.75) (end 136.75 61.5) (width 0.5) (layer "F.Cu") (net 10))
 (segment (start 133.5 64) (end 135.5 64) (width 0.5) (layer "F.Cu") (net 10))
 (segment (start 132.445 65.055) (end 133.5 64) (width 0.5) (layer "F.Cu") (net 10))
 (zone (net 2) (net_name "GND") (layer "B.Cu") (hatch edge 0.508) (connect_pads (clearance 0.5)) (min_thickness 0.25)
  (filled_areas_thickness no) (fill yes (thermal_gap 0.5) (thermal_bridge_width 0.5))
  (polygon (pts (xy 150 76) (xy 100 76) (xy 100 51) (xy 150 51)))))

